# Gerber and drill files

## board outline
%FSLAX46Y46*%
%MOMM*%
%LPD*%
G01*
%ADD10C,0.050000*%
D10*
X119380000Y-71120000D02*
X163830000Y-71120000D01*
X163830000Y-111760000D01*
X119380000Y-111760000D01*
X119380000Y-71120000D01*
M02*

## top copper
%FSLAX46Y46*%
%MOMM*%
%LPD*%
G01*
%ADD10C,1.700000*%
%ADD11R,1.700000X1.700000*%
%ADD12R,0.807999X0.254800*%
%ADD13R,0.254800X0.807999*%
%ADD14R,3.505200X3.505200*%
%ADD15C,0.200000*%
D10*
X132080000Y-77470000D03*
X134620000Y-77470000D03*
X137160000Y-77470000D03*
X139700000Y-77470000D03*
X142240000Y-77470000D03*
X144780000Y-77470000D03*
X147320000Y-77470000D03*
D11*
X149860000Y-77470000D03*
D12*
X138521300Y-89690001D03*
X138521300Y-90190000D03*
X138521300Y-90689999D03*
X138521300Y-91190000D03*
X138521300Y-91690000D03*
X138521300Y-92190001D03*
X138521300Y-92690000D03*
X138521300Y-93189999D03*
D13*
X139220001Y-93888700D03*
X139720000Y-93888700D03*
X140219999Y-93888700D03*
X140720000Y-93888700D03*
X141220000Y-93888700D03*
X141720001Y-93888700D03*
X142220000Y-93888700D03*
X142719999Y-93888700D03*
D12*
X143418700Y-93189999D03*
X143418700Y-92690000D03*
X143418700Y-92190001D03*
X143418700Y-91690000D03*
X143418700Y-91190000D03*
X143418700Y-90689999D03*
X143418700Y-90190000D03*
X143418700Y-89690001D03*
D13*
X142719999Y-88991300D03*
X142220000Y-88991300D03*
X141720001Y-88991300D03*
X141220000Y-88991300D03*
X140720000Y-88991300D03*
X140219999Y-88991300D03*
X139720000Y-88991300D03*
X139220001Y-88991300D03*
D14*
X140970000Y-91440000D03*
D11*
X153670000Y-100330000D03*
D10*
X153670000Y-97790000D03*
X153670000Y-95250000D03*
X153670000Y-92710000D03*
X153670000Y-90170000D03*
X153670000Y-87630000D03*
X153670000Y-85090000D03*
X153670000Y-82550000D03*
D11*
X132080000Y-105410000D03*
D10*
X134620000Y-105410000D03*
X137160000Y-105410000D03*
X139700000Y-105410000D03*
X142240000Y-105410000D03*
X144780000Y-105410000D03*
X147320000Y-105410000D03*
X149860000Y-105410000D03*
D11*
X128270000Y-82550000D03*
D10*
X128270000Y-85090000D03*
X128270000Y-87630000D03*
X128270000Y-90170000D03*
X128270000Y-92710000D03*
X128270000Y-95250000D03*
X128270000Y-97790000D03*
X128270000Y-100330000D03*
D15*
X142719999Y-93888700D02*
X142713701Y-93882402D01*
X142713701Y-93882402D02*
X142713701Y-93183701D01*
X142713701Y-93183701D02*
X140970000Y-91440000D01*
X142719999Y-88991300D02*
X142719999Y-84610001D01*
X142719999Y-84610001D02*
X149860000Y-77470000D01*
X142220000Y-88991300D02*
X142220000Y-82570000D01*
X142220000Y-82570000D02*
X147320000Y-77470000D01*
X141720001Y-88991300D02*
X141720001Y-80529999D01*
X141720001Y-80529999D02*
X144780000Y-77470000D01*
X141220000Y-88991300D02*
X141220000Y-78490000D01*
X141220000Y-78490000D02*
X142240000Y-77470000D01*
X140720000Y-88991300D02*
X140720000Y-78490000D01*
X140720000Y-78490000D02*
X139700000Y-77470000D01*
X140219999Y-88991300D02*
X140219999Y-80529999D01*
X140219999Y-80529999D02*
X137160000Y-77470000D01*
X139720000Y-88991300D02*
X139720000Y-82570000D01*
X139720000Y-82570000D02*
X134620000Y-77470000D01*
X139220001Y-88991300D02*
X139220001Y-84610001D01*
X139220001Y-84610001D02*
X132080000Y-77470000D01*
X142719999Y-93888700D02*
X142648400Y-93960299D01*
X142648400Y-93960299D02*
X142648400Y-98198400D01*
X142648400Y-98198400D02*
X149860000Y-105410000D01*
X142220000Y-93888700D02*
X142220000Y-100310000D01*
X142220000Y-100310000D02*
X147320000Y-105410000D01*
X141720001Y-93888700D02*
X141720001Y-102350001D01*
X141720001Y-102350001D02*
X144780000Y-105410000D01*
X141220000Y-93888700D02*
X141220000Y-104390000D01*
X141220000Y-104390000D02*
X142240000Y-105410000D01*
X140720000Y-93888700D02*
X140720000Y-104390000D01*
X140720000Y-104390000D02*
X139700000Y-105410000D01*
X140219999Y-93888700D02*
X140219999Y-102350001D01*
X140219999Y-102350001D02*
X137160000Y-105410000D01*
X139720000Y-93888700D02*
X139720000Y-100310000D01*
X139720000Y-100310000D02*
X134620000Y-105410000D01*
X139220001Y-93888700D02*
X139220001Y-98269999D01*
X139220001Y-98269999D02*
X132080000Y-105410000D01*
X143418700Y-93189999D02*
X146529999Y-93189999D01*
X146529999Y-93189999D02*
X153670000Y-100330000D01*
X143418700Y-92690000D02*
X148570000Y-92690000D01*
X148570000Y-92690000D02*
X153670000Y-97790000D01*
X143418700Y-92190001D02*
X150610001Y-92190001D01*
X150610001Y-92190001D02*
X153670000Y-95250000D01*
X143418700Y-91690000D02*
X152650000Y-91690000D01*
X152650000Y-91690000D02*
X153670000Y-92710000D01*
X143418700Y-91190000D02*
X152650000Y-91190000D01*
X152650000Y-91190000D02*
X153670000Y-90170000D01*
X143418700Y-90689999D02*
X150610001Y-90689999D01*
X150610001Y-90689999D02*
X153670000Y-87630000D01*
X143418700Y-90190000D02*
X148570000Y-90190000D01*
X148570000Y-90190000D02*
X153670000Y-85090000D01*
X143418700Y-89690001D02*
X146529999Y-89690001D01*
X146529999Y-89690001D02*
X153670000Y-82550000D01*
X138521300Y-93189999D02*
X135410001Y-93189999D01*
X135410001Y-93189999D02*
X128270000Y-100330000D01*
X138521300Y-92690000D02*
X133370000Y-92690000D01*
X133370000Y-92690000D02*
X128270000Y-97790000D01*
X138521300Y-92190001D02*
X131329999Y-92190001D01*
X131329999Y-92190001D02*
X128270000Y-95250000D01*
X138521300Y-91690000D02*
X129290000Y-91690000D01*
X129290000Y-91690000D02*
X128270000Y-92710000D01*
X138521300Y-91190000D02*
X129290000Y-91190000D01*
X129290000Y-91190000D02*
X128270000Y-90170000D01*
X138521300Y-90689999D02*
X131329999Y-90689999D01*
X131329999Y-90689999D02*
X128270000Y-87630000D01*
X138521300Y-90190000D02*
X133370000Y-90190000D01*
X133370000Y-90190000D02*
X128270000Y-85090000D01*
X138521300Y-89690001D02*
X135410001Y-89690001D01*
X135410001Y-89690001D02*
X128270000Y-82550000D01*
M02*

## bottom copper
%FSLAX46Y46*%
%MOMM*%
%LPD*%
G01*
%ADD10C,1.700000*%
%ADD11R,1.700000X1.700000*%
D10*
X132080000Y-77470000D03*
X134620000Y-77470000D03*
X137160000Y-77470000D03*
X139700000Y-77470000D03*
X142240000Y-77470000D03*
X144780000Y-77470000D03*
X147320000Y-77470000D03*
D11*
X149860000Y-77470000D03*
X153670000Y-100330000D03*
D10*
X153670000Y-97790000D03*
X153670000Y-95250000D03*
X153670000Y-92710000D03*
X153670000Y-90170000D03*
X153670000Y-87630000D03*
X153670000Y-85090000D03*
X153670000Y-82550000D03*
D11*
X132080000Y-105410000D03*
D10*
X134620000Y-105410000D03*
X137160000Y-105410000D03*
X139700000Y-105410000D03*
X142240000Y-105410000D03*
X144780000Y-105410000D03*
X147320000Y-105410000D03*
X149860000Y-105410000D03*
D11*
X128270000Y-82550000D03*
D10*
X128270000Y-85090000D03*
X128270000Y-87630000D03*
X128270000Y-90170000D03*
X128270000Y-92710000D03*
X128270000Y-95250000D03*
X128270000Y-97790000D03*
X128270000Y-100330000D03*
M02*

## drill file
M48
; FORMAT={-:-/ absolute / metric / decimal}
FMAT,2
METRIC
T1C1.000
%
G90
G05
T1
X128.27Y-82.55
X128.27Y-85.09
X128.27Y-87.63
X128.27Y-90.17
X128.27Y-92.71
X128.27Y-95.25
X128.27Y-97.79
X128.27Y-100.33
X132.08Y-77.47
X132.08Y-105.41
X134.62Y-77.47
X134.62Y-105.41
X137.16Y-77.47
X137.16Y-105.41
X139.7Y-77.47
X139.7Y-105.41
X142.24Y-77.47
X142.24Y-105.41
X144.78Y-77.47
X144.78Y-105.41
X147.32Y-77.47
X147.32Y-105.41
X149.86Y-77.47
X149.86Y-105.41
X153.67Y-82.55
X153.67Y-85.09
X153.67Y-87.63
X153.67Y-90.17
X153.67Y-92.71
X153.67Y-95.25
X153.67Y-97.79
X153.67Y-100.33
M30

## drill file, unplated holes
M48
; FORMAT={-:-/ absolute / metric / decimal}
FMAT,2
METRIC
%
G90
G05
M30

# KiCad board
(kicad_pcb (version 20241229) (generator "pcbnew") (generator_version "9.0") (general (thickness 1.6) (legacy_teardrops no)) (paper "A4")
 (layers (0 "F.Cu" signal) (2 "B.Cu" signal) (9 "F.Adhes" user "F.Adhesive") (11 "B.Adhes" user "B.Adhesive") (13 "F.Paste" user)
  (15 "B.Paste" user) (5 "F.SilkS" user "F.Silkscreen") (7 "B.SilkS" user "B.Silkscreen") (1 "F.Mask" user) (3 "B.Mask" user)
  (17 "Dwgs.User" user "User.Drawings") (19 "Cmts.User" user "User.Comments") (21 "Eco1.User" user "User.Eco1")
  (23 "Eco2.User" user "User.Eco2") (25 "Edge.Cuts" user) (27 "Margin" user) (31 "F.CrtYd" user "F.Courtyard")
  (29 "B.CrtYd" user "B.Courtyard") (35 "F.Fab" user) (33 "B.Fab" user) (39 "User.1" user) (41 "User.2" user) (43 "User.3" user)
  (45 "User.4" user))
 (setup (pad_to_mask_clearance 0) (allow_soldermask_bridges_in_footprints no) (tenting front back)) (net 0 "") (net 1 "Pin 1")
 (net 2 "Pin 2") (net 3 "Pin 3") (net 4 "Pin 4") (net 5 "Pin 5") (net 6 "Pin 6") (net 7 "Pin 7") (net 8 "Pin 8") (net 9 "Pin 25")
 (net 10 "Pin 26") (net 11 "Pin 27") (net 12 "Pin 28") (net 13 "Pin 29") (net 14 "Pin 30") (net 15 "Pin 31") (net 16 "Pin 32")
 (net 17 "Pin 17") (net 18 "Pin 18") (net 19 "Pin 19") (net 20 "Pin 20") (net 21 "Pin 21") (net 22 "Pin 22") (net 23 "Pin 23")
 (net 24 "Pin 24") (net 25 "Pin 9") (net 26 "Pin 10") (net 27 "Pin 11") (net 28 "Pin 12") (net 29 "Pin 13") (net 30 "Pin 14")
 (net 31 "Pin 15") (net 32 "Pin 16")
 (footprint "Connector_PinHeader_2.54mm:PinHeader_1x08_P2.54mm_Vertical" (layer "F.Cu") (at 128.27 82.55)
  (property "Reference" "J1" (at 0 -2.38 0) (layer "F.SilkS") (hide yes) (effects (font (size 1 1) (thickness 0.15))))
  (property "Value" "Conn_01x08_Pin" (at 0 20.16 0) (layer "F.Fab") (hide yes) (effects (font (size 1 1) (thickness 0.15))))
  (pad "1" thru_hole rect (at 0 0) (size 1.7 1.7) (drill 1) (layers "*.Cu" "*.Mask") (remove_unused_layers no) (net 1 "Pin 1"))
  (pad "2" thru_hole circle (at 0 2.54) (size 1.7 1.7) (drill 1) (layers "*.Cu" "*.Mask") (remove_unused_layers no) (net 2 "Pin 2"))
  (pad "3" thru_hole circle (at 0 5.08) (size 1.7 1.7) (drill 1) (layers "*.Cu" "*.Mask") (remove_unused_layers no) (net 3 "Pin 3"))
  (pad "4" thru_hole circle (at 0 7.62) (size 1.7 1.7) (drill 1) (layers "*.Cu" "*.Mask") (remove_unused_layers no) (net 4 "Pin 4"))
  (pad "5" thru_hole circle (at 0 10.16) (size 1.7 1.7) (drill 1) (layers "*.Cu" "*.Mask") (remove_unused_layers no) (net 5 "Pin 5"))
  (pad "6" thru_hole circle (at 0 12.7) (size 1.7 1.7) (drill 1) (layers "*.Cu" "*.Mask") (remove_unused_layers no) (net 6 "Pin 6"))
  (pad "7" thru_hole circle (at 0 15.24) (size 1.7 1.7) (drill 1) (layers "*.Cu" "*.Mask") (remove_unused_layers no) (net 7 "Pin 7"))
  (pad "8" thru_hole circle (at 0 17.78) (size 1.7 1.7) (drill 1) (layers "*.Cu" "*.Mask") (remove_unused_layers no) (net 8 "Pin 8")))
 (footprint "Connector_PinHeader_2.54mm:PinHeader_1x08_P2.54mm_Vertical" (layer "F.Cu") (at 149.86 77.47 -90)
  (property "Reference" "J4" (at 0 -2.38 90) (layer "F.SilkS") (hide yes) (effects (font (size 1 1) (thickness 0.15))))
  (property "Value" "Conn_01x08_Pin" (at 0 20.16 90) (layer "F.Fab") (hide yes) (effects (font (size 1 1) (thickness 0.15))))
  (pad "1" thru_hole rect (at 0 0 270) (size 1.7 1.7) (drill 1) (layers "*.Cu" "*.Mask") (remove_unused_layers no) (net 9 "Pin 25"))
  (pad "2" thru_hole circle (at 0 2.54 270) (size 1.7 1.7) (drill 1) (layers "*.Cu" "*.Mask") (remove_unused_layers no) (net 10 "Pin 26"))
  (pad "3" thru_hole circle (at 0 5.08 270) (size 1.7 1.7) (drill 1) (layers "*.Cu" "*.Mask") (remove_unused_layers no) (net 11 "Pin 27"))
  (pad "4" thru_hole circle (at 0 7.62 270) (size 1.7 1.7) (drill 1) (layers "*.Cu" "*.Mask") (remove_unused_layers no) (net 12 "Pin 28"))
  (pad "5" thru_hole circle (at 0 10.16 270) (size 1.7 1.7) (drill 1) (layers "*.Cu" "*.Mask") (remove_unused_layers no) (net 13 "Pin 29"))
  (pad "6" thru_hole circle (at 0 12.7 270) (size 1.7 1.7) (drill 1) (layers "*.Cu" "*.Mask") (remove_unused_layers no) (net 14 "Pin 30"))
  (pad "7" thru_hole circle (at 0 15.24 270) (size 1.7 1.7) (drill 1) (layers "*.Cu" "*.Mask") (remove_unused_layers no) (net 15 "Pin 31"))
  (pad "8" thru_hole circle (at 0 17.78 270) (size 1.7 1.7) (drill 1) (layers "*.Cu" "*.Mask") (remove_unused_layers no) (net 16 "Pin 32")))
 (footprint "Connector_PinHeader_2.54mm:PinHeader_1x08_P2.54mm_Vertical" (layer "F.Cu") (at 153.67 100.33 180)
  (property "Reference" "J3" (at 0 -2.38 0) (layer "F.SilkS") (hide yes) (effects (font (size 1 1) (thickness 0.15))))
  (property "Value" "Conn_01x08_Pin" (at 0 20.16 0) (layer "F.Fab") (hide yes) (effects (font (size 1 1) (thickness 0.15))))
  (pad "1" thru_hole rect (at 0 0 180) (size 1.7 1.7) (drill 1) (layers "*.Cu" "*.Mask") (remove_unused_layers no) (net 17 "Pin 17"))
  (pad "2" thru_hole circle (at 0 2.54 180) (size 1.7 1.7) (drill 1) (layers "*.Cu" "*.Mask") (remove_unused_layers no) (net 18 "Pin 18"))
  (pad "3" thru_hole circle (at 0 5.08 180) (size 1.7 1.7) (drill 1) (layers "*.Cu" "*.Mask") (remove_unused_layers no) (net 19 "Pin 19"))
  (pad "4" thru_hole circle (at 0 7.62 180) (size 1.7 1.7) (drill 1) (layers "*.Cu" "*.Mask") (remove_unused_layers no) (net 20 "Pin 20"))
  (pad "5" thru_hole circle (at 0 10.16 180) (size 1.7 1.7) (drill 1) (layers "*.Cu" "*.Mask") (remove_unused_layers no) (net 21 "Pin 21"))
  (pad "6" thru_hole circle (at 0 12.7 180) (size 1.7 1.7) (drill 1) (layers "*.Cu" "*.Mask") (remove_unused_layers no) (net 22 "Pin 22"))
  (pad "7" thru_hole circle (at 0 15.24 180) (size 1.7 1.7) (drill 1) (layers "*.Cu" "*.Mask") (remove_unused_layers no) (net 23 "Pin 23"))
  (pad "8" thru_hole circle (at 0 17.78 180) (size 1.7 1.7) (drill 1) (layers "*.Cu" "*.Mask") (remove_unused_layers no) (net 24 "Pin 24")))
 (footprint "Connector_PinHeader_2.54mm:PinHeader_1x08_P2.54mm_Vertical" (layer "F.Cu") (at 132.08 105.41 90)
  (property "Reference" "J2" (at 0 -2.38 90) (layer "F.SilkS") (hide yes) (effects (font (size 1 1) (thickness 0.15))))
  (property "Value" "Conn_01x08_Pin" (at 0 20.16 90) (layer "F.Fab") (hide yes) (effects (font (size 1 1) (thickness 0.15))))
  (pad "1" thru_hole rect (at 0 0 90) (size 1.7 1.7) (drill 1) (layers "*.Cu" "*.Mask") (remove_unused_layers no) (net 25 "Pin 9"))
  (pad "2" thru_hole circle (at 0 2.54 90) (size 1.7 1.7) (drill 1) (layers "*.Cu" "*.Mask") (remove_unused_layers no) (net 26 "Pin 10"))
  (pad "3" thru_hole circle (at 0 5.08 90) (size 1.7 1.7) (drill 1) (layers "*.Cu" "*.Mask") (remove_unused_layers no) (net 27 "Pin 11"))
  (pad "4" thru_hole circle (at 0 7.62 90) (size 1.7 1.7) (drill 1) (layers "*.Cu" "*.Mask") (remove_unused_layers no) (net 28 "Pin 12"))
  (pad "5" thru_hole circle (at 0 10.16 90) (size 1.7 1.7) (drill 1) (layers "*.Cu" "*.Mask") (remove_unused_layers no) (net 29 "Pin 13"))
  (pad "6" thru_hole circle (at 0 12.7 90) (size 1.7 1.7) (drill 1) (layers "*.Cu" "*.Mask") (remove_unused_layers no) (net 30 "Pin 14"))
  (pad "7" thru_hole circle (at 0 15.24 90) (size 1.7 1.7) (drill 1) (layers "*.Cu" "*.Mask") (remove_unused_layers no) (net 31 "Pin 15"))
  (pad "8" thru_hole circle (at 0 17.78 90) (size 1.7 1.7) (drill 1) (layers "*.Cu" "*.Mask") (remove_unused_layers no) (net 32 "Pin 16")))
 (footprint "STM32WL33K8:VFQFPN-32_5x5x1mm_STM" (layer "F.Cu") (at 140.97 91.44)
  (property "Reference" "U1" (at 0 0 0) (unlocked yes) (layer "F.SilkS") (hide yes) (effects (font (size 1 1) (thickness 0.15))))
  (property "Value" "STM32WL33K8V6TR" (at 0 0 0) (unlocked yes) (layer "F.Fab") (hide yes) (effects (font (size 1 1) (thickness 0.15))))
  (pad "1" smd rect (at -2.4487 -1.749999 90) (size 0.2548 0.807999) (layers "F.Cu" "F.Mask" "F.Paste") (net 1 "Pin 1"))
  (pad "2" smd rect (at -2.4487 -1.25 90) (size 0.2548 0.807999) (layers "F.Cu" "F.Mask" "F.Paste") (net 2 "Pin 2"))
  (pad "3" smd rect (at -2.4487 -0.750001 90) (size 0.2548 0.807999) (layers "F.Cu" "F.Mask" "F.Paste") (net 3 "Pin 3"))
  (pad "4" smd rect (at -2.4487 -0.25 90) (size 0.2548 0.807999) (layers "F.Cu" "F.Mask" "F.Paste") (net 4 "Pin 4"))
  (pad "5" smd rect (at -2.4487 0.25 90) (size 0.2548 0.807999) (layers "F.Cu" "F.Mask" "F.Paste") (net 5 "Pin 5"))
  (pad "6" smd rect (at -2.4487 0.750001 90) (size 0.2548 0.807999) (layers "F.Cu" "F.Mask" "F.Paste") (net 6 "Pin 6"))
  (pad "7" smd rect (at -2.4487 1.25 90) (size 0.2548 0.807999) (layers "F.Cu" "F.Mask" "F.Paste") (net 7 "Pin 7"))
  (pad "8" smd rect (at -2.4487 1.749999 90) (size 0.2548 0.807999) (layers "F.Cu" "F.Mask" "F.Paste") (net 8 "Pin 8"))
  (pad "9" smd rect (at -1.749999 2.4487) (size 0.2548 0.807999) (layers "F.Cu" "F.Mask" "F.Paste") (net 25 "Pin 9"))
  (pad "10" smd rect (at -1.25 2.4487) (size 0.2548 0.807999) (layers "F.Cu" "F.Mask" "F.Paste") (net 26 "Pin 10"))
  (pad "11" smd rect (at -0.750001 2.4487) (size 0.2548 0.807999) (layers "F.Cu" "F.Mask" "F.Paste") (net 27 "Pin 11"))
  (pad "12" smd rect (at -0.25 2.4487) (size 0.2548 0.807999) (layers "F.Cu" "F.Mask" "F.Paste") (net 28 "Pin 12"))
  (pad "13" smd rect (at 0.25 2.4487) (size 0.2548 0.807999) (layers "F.Cu" "F.Mask" "F.Paste") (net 29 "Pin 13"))
  (pad "14" smd rect (at 0.750001 2.4487) (size 0.2548 0.807999) (layers "F.Cu" "F.Mask" "F.Paste") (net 30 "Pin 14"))
  (pad "15" smd rect (at 1.25 2.4487) (size 0.2548 0.807999) (layers "F.Cu" "F.Mask" "F.Paste") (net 31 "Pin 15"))
  (pad "16" smd rect (at 1.749999 2.4487) (size 0.2548 0.807999) (layers "F.Cu" "F.Mask" "F.Paste") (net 32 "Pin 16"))
  (pad "17" smd rect (at 2.4487 1.749999 90) (size 0.2548 0.807999) (layers "F.Cu" "F.Mask" "F.Paste") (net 17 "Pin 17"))
  (pad "18" smd rect (at 2.4487 1.25 90) (size 0.2548 0.807999) (layers "F.Cu" "F.Mask" "F.Paste") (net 18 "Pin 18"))
  (pad "19" smd rect (at 2.4487 0.750001 90) (size 0.2548 0.807999) (layers "F.Cu" "F.Mask" "F.Paste") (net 19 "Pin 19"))
  (pad "20" smd rect (at 2.4487 0.25 90) (size 0.2548 0.807999) (layers "F.Cu" "F.Mask" "F.Paste") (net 20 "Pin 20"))
  (pad "21" smd rect (at 2.4487 -0.25 90) (size 0.2548 0.807999) (layers "F.Cu" "F.Mask" "F.Paste") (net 21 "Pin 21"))
  (pad "22" smd rect (at 2.4487 -0.750001 90) (size 0.2548 0.807999) (layers "F.Cu" "F.Mask" "F.Paste") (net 22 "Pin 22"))
  (pad "23" smd rect (at 2.4487 -1.25 90) (size 0.2548 0.807999) (layers "F.Cu" "F.Mask" "F.Paste") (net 23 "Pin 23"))
  (pad "24" smd rect (at 2.4487 -1.749999 90) (size 0.2548 0.807999) (layers "F.Cu" "F.Mask" "F.Paste") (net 24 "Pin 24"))
  (pad "25" smd rect (at 1.749999 -2.4487) (size 0.2548 0.807999) (layers "F.Cu" "F.Mask" "F.Paste") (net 9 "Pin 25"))
  (pad "26" smd rect (at 1.25 -2.4487) (size 0.2548 0.807999) (layers "F.Cu" "F.Mask" "F.Paste") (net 10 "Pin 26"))
  (pad "27" smd rect (at 0.750001 -2.4487) (size 0.2548 0.807999) (layers "F.Cu" "F.Mask" "F.Paste") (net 11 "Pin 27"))
  (pad "28" smd rect (at 0.25 -2.4487) (size 0.2548 0.807999) (layers "F.Cu" "F.Mask" "F.Paste") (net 12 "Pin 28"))
  (pad "29" smd rect (at -0.25 -2.4487) (size 0.2548 0.807999) (layers "F.Cu" "F.Mask" "F.Paste") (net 13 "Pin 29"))
  (pad "30" smd rect (at -0.750001 -2.4487) (size 0.2548 0.807999) (layers "F.Cu" "F.Mask" "F.Paste") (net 14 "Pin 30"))
  (pad "31" smd rect (at -1.25 -2.4487) (size 0.2548 0.807999) (layers "F.Cu" "F.Mask" "F.Paste") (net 15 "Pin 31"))
  (pad "32" smd rect (at -1.749999 -2.4487) (size 0.2548 0.807999) (layers "F.Cu" "F.Mask" "F.Paste") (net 16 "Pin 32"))
  (pad "33" smd rect (at 0 0) (size 3.5052 3.5052) (layers "F.Cu" "F.Mask" "F.Paste") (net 32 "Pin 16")))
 (gr_rect (start 119.38 71.12) (end 163.83 111.76) (stroke (width 0.05) (type default)) (fill no) (layer "Edge.Cuts"))
 (segment (start 138.5213 93.189999) (end 135.410001 93.189999) (width 0.2) (layer "F.Cu") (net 8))
 (segment (start 135.410001 93.189999) (end 128.27 100.33) (width 0.2) (layer "F.Cu") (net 8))
 (segment (start 135.410001 89.690001) (end 128.27 82.55) (width 0.2) (layer "F.Cu") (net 1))
 (segment (start 138.5213 89.690001) (end 135.410001 89.690001) (width 0.2) (layer "F.Cu") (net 1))
 (segment (start 133.37 92.69) (end 128.27 97.79) (width 0.2) (layer "F.Cu") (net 7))
 (segment (start 138.5213 92.69) (end 133.37 92.69) (width 0.2) (layer "F.Cu") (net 7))
 (segment (start 133.37 90.19) (end 128.27 85.09) (width 0.2) (layer "F.Cu") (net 2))
 (segment (start 138.5213 90.19) (end 133.37 90.19) (width 0.2) (layer "F.Cu") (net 2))
 (segment (start 138.5213 91.19) (end 129.29 91.19) (width 0.2) (layer "F.Cu") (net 4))
 (segment (start 129.29 91.19) (end 128.27 90.17) (width 0.2) (layer "F.Cu") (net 4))
 (segment (start 138.5213 90.689999) (end 131.329999 90.689999) (width 0.2) (layer "F.Cu") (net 3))
 (segment (start 131.329999 90.689999) (end 128.27 87.63) (width 0.2) (layer "F.Cu") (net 3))
 (segment (start 138.5213 92.190001) (end 131.329999 92.190001) (width 0.2) (layer "F.Cu") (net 6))
 (segment (start 131.329999 92.190001) (end 128.27 95.25) (width 0.2) (layer "F.Cu") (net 6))
 (segment (start 138.5213 91.69) (end 129.29 91.69) (width 0.2) (layer "F.Cu") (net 5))
 (segment (start 129.29 91.69) (end 128.27 92.71) (width 0.2) (layer "F.Cu") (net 5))
 (segment (start 142.719999 93.8887) (end 142.713701 93.882402) (width 0.2) (layer "F.Cu") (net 32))
 (segment (start 142.713701 93.882402) (end 142.713701 93.183701) (width 0.2) (layer "F.Cu") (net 32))
 (segment (start 142.713701 93.183701) (end 140.97 91.44) (width 0.2) (layer "F.Cu") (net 32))
 (segment (start 142.6484 98.1984) (end 149.86 105.41) (width 0.2) (layer "F.Cu") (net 32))
 (segment (start 142.719999 93.8887) (end 142.6484 93.960299) (width 0.2) (layer "F.Cu") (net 32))
 (segment (start 142.6484 93.960299) (end 142.6484 98.1984) (width 0.2) (layer "F.Cu") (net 32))
 (segment (start 141.22 104.39) (end 142.24 105.41) (width 0.2) (layer "F.Cu") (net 29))
 (segment (start 141.22 93.8887) (end 141.22 104.39) (width 0.2) (layer "F.Cu") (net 29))
 (segment (start 142.22 93.8887) (end 142.22 100.31) (width 0.2) (layer "F.Cu") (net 31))
 (segment (start 142.22 100.31) (end 147.32 105.41) (width 0.2) (layer "F.Cu") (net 31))
 (segment (start 139.220001 98.269999) (end 132.08 105.41) (width 0.2) (layer "F.Cu") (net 25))
 (segment (start 139.220001 93.8887) (end 139.220001 98.269999) (width 0.2) (layer "F.Cu") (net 25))
 (segment (start 139.72 93.8887) (end 139.72 100.31) (width 0.2) (layer "F.Cu") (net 26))
 (segment (start 139.72 100.31) (end 134.62 105.41) (width 0.2) (layer "F.Cu") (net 26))
 (segment (start 141.720001 93.8887) (end 141.720001 102.350001) (width 0.2) (layer "F.Cu") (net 30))
 (segment (start 141.720001 102.350001) (end 144.78 105.41) (width 0.2) (layer "F.Cu") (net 30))
 (segment (start 140.72 104.39) (end 139.7 105.41) (width 0.2) (layer "F.Cu") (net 28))
 (segment (start 140.72 93.8887) (end 140.72 104.39) (width 0.2) (layer "F.Cu") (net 28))
 (segment (start 140.219999 93.8887) (end 140.219999 102.350001) (width 0.2) (layer "F.Cu") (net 27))
 (segment (start 140.219999 102.350001) (end 137.16 105.41) (width 0.2) (layer "F.Cu") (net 27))
 (segment (start 143.4187 90.19) (end 148.57 90.19) (width 0.2) (layer "F.Cu") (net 23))
 (segment (start 148.57 90.19) (end 153.67 85.09) (width 0.2) (layer "F.Cu") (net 23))
 (segment (start 143.4187 93.189999) (end 146.529999 93.189999) (width 0.2) (layer "F.Cu") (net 17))
 (segment (start 146.529999 93.189999) (end 153.67 100.33) (width 0.2) (layer "F.Cu") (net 17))
 (segment (start 150.610001 92.190001) (end 153.67 95.25) (width 0.2) (layer "F.Cu") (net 19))
 (segment (start 143.4187 92.190001) (end 150.610001 92.190001) (width 0.2) (layer "F.Cu") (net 19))
 (segment (start 143.4187 92.69) (end 148.57 92.69) (width 0.2) (layer "F.Cu") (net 18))
 (segment (start 148.57 92.69) (end 153.67 97.79) (width 0.2) (layer "F.Cu") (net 18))
 (segment (start 152.65 91.19) (end 153.67 90.17) (width 0.2) (layer "F.Cu") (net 21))
 (segment (start 143.4187 91.19) (end 152.65 91.19) (width 0.2) (layer "F.Cu") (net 21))
 (segment (start 146.529999 89.690001) (end 153.67 82.55) (width 0.2) (layer "F.Cu") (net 24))
 (segment (start 143.4187 89.690001) (end 146.529999 89.690001) (width 0.2) (layer "F.Cu") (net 24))
 (segment (start 150.610001 90.689999) (end 153.67 87.63) (width 0.2) (layer "F.Cu") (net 22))
 (segment (start 143.4187 90.689999) (end 150.610001 90.689999) (width 0.2) (layer "F.Cu") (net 22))
 (segment (start 152.65 91.69) (end 153.67 92.71) (width 0.2) (layer "F.Cu") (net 20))
 (segment (start 143.4187 91.69) (end 152.65 91.69) (width 0.2) (layer "F.Cu") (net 20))
 (segment (start 142.719999 84.610001) (end 149.86 77.47) (width 0.2) (layer "F.Cu") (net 9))
 (segment (start 142.719999 88.9913) (end 142.719999 84.610001) (width 0.2) (layer "F.Cu") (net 9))
 (segment (start 141.22 88.9913) (end 141.22 78.49) (width 0.2) (layer "F.Cu") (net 12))
 (segment (start 141.22 78.49) (end 142.24 77.47) (width 0.2) (layer "F.Cu") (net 12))
 (segment (start 140.72 88.9913) (end 140.72 78.49) (width 0.2) (layer "F.Cu") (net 13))
 (segment (start 140.72 78.49) (end 139.7 77.47) (width 0.2) (layer "F.Cu") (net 13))
 (segment (start 139.72 88.9913) (end 139.72 82.57) (width 0.2) (layer "F.Cu") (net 15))
 (segment (start 139.72 82.57) (end 134.62 77.47) (width 0.2) (layer "F.Cu") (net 15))
 (segment (start 140.219999 88.9913) (end 140.219999 80.529999) (width 0.2) (layer "F.Cu") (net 14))
 (segment (start 140.219999 80.529999) (end 137.16 77.47) (width 0.2) (layer "F.Cu") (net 14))
 (segment (start 142.22 82.57) (end 147.32 77.47) (width 0.2) (layer "F.Cu") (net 10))
 (segment (start 142.22 88.9913) (end 142.22 82.57) (width 0.2) (layer "F.Cu") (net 10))
 (segment (start 141.720001 88.9913) (end 141.720001 80.529999) (width 0.2) (layer "F.Cu") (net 11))
 (segment (start 141.720001 80.529999) (end 144.78 77.47) (width 0.2) (layer "F.Cu") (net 11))
 (segment (start 139.220001 84.610001) (end 132.08 77.47) (width 0.2) (layer "F.Cu") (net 16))
 (segment (start 139.220001 88.9913) (end 139.220001 84.610001) (width 0.2) (layer "F.Cu") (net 16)))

